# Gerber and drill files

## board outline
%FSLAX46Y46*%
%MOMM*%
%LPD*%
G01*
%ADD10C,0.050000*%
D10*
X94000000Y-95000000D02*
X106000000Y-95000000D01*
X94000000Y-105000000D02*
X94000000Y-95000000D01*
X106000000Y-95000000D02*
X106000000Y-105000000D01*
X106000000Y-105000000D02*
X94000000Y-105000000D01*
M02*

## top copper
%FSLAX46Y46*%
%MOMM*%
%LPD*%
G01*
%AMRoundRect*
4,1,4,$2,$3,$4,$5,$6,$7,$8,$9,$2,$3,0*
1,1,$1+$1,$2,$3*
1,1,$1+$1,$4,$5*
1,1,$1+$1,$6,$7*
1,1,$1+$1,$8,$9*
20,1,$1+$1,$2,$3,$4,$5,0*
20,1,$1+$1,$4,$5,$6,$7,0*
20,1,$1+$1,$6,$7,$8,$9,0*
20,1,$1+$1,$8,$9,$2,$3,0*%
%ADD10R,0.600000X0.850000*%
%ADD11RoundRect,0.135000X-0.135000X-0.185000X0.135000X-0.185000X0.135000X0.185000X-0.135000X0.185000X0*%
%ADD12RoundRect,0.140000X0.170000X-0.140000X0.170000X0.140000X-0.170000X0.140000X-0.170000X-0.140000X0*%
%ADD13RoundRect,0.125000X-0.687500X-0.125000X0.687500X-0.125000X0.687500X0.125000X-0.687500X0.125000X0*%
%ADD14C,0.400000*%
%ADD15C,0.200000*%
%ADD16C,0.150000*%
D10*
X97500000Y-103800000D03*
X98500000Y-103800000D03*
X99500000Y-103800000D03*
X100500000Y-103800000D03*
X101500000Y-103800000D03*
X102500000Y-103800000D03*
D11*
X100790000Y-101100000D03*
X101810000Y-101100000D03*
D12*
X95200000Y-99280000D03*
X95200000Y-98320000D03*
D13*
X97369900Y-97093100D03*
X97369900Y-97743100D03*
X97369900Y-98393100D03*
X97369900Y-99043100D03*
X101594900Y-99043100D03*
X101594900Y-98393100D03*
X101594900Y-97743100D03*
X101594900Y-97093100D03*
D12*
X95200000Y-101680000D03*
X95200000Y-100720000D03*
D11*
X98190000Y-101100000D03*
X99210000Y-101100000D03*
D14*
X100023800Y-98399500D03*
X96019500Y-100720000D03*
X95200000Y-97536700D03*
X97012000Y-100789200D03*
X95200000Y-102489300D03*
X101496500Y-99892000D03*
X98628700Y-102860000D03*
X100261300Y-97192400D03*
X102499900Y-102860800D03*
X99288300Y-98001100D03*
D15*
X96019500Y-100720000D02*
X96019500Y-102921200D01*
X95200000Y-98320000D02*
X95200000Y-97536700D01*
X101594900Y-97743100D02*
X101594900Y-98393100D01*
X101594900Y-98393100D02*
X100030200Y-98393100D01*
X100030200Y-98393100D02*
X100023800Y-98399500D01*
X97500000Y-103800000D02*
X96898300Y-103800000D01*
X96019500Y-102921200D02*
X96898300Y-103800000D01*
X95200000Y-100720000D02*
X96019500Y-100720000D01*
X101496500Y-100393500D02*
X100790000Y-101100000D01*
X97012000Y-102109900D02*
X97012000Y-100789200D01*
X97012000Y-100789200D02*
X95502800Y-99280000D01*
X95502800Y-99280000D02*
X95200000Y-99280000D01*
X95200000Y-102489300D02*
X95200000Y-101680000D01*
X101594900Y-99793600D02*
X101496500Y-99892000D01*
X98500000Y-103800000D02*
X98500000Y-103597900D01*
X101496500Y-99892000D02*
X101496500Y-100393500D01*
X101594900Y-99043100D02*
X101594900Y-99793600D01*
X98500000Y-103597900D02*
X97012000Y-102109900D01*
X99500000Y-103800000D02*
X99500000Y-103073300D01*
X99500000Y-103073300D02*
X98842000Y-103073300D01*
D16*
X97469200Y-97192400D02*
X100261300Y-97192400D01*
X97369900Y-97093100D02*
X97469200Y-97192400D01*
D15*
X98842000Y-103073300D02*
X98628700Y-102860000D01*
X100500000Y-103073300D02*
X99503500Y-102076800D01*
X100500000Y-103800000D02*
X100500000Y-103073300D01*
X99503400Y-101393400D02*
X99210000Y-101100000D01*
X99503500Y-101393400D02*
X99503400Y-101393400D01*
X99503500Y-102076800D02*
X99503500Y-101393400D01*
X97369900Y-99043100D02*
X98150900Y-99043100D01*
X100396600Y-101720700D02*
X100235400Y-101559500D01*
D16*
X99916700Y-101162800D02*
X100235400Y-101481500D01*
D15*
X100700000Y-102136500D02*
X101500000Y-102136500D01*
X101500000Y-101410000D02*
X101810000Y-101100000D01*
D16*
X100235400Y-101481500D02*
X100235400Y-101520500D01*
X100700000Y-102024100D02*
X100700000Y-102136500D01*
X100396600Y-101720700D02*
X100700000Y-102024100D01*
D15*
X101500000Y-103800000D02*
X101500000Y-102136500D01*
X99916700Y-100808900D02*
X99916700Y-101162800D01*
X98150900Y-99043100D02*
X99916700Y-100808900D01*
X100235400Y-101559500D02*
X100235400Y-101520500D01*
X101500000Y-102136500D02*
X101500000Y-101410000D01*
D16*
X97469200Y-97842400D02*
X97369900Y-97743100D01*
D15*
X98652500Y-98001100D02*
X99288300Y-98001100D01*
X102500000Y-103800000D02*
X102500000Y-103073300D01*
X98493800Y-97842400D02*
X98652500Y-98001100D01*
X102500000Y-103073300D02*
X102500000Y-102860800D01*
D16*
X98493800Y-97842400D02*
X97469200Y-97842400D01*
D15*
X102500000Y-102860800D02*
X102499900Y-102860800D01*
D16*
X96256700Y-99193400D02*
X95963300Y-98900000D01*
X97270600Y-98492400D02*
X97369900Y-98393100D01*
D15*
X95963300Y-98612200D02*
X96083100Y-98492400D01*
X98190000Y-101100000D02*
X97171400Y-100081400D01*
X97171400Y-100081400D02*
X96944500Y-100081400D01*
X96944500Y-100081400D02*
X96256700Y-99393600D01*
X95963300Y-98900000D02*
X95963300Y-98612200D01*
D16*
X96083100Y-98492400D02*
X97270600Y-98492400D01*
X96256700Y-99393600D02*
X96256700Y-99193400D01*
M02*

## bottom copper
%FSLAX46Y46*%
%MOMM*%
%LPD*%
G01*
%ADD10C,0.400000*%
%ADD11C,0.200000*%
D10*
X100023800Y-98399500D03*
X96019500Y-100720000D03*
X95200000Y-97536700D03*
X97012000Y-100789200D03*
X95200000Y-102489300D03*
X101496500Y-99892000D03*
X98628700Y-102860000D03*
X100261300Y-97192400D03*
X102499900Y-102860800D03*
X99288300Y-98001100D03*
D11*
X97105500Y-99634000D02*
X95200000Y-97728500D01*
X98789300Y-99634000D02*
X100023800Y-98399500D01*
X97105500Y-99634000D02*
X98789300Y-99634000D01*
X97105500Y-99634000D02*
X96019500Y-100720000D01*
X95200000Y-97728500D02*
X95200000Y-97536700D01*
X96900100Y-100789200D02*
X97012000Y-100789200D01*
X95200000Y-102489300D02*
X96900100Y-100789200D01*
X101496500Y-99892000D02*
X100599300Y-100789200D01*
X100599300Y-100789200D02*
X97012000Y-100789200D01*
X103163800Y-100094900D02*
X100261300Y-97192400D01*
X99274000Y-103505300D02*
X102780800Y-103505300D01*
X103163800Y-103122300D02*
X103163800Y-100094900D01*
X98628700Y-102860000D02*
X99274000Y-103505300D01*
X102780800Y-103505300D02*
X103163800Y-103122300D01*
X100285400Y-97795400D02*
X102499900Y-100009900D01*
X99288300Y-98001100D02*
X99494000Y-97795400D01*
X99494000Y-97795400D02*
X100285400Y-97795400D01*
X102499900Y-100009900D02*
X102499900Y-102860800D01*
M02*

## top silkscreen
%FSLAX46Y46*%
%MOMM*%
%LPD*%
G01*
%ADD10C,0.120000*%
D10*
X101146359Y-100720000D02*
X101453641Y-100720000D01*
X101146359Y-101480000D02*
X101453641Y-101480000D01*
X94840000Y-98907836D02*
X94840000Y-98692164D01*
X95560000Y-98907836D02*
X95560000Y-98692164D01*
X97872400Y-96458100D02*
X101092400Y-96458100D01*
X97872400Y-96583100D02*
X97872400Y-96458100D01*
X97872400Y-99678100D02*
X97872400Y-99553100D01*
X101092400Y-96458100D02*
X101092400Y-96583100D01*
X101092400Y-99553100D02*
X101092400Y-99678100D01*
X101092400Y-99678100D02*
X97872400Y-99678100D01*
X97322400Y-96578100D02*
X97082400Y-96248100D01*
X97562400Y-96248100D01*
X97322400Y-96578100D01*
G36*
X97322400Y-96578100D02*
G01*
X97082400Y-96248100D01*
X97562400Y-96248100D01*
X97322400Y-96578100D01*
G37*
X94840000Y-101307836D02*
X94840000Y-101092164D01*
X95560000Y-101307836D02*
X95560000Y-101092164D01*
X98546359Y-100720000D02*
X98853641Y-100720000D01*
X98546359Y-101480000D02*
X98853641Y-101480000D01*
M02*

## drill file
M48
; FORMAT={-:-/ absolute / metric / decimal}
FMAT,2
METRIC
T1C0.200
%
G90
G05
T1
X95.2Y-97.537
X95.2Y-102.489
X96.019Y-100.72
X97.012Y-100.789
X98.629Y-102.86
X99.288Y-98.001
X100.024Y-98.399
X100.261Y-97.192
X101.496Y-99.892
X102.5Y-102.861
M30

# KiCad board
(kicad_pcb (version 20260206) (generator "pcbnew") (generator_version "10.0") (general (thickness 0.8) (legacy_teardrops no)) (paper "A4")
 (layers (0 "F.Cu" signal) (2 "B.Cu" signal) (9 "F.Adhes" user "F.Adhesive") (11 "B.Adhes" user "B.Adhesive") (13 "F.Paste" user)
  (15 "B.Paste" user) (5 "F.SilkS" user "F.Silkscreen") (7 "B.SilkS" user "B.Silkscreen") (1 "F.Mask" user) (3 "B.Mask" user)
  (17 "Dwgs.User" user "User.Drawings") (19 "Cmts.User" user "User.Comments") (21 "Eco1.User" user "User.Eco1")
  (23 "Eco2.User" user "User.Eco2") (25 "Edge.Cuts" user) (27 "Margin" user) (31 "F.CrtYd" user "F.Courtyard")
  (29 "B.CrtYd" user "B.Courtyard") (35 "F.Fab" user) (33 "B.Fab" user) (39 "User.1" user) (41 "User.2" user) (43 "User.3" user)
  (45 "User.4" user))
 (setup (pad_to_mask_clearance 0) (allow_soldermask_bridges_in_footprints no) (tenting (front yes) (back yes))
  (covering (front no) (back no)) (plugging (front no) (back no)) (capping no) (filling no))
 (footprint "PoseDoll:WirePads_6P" (layer "F.Cu") (at 100 103.8)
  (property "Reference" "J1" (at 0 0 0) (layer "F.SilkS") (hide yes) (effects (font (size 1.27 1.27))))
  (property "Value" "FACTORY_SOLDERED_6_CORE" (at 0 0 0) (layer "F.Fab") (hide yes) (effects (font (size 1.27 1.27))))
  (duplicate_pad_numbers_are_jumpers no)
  (pad "1" smd rect (at -2.5 0) (size 0.6 0.85) (layers "F.Cu" "F.Mask") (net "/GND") (thermal_bridge_angle 45))
  (pad "2" smd rect (at -1.5 0) (size 0.6 0.85) (layers "F.Cu" "F.Mask") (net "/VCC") (thermal_bridge_angle 45))
  (pad "3" smd rect (at -0.5 0) (size 0.6 0.85) (layers "F.Cu" "F.Mask") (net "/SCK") (thermal_bridge_angle 45))
  (pad "4" smd rect (at 0.5 0) (size 0.6 0.85) (layers "F.Cu" "F.Mask") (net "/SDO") (thermal_bridge_angle 45))
  (pad "5" smd rect (at 1.5 0) (size 0.6 0.85) (layers "F.Cu" "F.Mask") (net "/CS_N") (thermal_bridge_angle 45))
  (pad "6" smd rect (at 2.5 0) (size 0.6 0.85) (layers "F.Cu" "F.Mask") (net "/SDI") (thermal_bridge_angle 45)))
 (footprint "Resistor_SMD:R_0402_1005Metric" (layer "F.Cu") (at 101.3 101.1)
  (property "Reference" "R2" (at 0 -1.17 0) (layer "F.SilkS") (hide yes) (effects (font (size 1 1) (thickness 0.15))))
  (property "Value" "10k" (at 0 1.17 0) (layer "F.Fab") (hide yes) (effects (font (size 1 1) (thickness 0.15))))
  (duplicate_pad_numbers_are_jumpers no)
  (fp_line (start -0.153641 -0.38) (end 0.153641 -0.38) (stroke (width 0.12) (type solid)) (layer "F.SilkS"))
  (fp_line (start -0.153641 0.38) (end 0.153641 0.38) (stroke (width 0.12) (type solid)) (layer "F.SilkS"))
  (pad "1" smd roundrect (at -0.51 0) (size 0.54 0.64) (layers "F.Cu" "F.Mask" "F.Paste") (roundrect_rratio 0.25) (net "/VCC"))
  (pad "2" smd roundrect (at 0.51 0) (size 0.54 0.64) (layers "F.Cu" "F.Mask" "F.Paste") (roundrect_rratio 0.25) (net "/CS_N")))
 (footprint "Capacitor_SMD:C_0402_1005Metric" (layer "F.Cu") (at 95.2 98.8 90)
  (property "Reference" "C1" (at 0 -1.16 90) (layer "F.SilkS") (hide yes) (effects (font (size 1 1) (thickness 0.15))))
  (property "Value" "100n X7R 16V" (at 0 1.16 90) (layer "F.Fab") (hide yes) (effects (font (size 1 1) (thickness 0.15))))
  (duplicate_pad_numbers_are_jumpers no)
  (fp_line (start -0.107836 -0.36) (end 0.107836 -0.36) (stroke (width 0.12) (type solid)) (layer "F.SilkS"))
  (fp_line (start -0.107836 0.36) (end 0.107836 0.36) (stroke (width 0.12) (type solid)) (layer "F.SilkS"))
  (pad "1" smd roundrect (at -0.48 0 90) (size 0.56 0.62) (layers "F.Cu" "F.Mask" "F.Paste") (roundrect_rratio 0.25) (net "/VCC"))
  (pad "2" smd roundrect (at 0.48 0 90) (size 0.56 0.62) (layers "F.Cu" "F.Mask" "F.Paste") (roundrect_rratio 0.25) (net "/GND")))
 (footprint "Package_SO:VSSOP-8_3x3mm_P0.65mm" (layer "F.Cu") (at 99.4824 98.0681)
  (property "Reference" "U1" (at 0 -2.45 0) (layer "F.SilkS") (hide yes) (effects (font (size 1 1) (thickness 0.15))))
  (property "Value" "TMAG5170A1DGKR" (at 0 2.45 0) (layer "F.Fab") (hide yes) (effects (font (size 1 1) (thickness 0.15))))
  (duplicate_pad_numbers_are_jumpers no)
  (fp_line (start -1.61 -1.61) (end 1.61 -1.61) (stroke (width 0.12) (type solid)) (layer "F.SilkS"))
  (fp_line (start -1.61 -1.485) (end -1.61 -1.61) (stroke (width 0.12) (type solid)) (layer "F.SilkS"))
  (fp_line (start -1.61 1.61) (end -1.61 1.485) (stroke (width 0.12) (type solid)) (layer "F.SilkS"))
  (fp_line (start 1.61 -1.61) (end 1.61 -1.485) (stroke (width 0.12) (type solid)) (layer "F.SilkS"))
  (fp_line (start 1.61 1.485) (end 1.61 1.61) (stroke (width 0.12) (type solid)) (layer "F.SilkS"))
  (fp_line (start 1.61 1.61) (end -1.61 1.61) (stroke (width 0.12) (type solid)) (layer "F.SilkS"))
  (fp_poly (pts (xy -2.16 -1.49) (xy -2.4 -1.82) (xy -1.92 -1.82)) (stroke (width 0.12) (type solid)) (fill yes) (layer "F.SilkS"))
  (pad "1" smd roundrect (at -2.1125 -0.975) (size 1.625 0.5) (layers "F.Cu" "F.Mask" "F.Paste") (roundrect_rratio 0.25) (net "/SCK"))
  (pad "2" smd roundrect (at -2.1125 -0.325) (size 1.625 0.5) (layers "F.Cu" "F.Mask" "F.Paste") (roundrect_rratio 0.25) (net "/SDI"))
  (pad "3" smd roundrect (at -2.1125 0.325) (size 1.625 0.5) (layers "F.Cu" "F.Mask" "F.Paste") (roundrect_rratio 0.25) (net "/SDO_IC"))
  (pad "4" smd roundrect (at -2.1125 0.975) (size 1.625 0.5) (layers "F.Cu" "F.Mask" "F.Paste") (roundrect_rratio 0.25) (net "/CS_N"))
  (pad "5" smd roundrect (at 2.1125 0.975) (size 1.625 0.5) (layers "F.Cu" "F.Mask" "F.Paste") (roundrect_rratio 0.25) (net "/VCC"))
  (pad "6" smd roundrect (at 2.1125 0.325) (size 1.625 0.5) (layers "F.Cu" "F.Mask" "F.Paste") (roundrect_rratio 0.25) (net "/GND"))
  (pad "7" smd roundrect (at 2.1125 -0.325) (size 1.625 0.5) (layers "F.Cu" "F.Mask" "F.Paste") (roundrect_rratio 0.25) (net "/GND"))
  (pad "8" smd roundrect (at 2.1125 -0.975) (size 1.625 0.5) (layers "F.Cu" "F.Mask" "F.Paste") (roundrect_rratio 0.25)
   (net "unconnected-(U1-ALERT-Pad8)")))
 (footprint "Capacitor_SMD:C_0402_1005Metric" (layer "F.Cu") (at 95.2 101.2 90)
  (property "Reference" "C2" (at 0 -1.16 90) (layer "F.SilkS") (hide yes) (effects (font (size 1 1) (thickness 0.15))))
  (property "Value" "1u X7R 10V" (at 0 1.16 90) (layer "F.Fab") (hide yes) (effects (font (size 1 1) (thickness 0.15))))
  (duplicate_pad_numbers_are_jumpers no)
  (fp_line (start -0.107836 -0.36) (end 0.107836 -0.36) (stroke (width 0.12) (type solid)) (layer "F.SilkS"))
  (fp_line (start -0.107836 0.36) (end 0.107836 0.36) (stroke (width 0.12) (type solid)) (layer "F.SilkS"))
  (pad "1" smd roundrect (at -0.48 0 90) (size 0.56 0.62) (layers "F.Cu" "F.Mask" "F.Paste") (roundrect_rratio 0.25) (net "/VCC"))
  (pad "2" smd roundrect (at 0.48 0 90) (size 0.56 0.62) (layers "F.Cu" "F.Mask" "F.Paste") (roundrect_rratio 0.25) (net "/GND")))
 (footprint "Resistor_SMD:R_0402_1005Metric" (layer "F.Cu") (at 98.7 101.1)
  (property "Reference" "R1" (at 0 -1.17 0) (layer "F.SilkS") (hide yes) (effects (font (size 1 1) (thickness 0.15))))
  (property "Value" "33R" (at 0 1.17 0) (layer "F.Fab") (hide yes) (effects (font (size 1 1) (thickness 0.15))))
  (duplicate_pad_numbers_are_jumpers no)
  (fp_line (start -0.153641 -0.38) (end 0.153641 -0.38) (stroke (width 0.12) (type solid)) (layer "F.SilkS"))
  (fp_line (start -0.153641 0.38) (end 0.153641 0.38) (stroke (width 0.12) (type solid)) (layer "F.SilkS"))
  (pad "1" smd roundrect (at -0.51 0) (size 0.54 0.64) (layers "F.Cu" "F.Mask" "F.Paste") (roundrect_rratio 0.25) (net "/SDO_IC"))
  (pad "2" smd roundrect (at 0.51 0) (size 0.54 0.64) (layers "F.Cu" "F.Mask" "F.Paste") (roundrect_rratio 0.25) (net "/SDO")))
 (gr_line (start 94 95) (end 106 95) (stroke (width 0.05) (type default)) (layer "Edge.Cuts"))
 (gr_line (start 94 105) (end 94 95) (stroke (width 0.05) (type default)) (layer "Edge.Cuts"))
 (gr_line (start 106 95) (end 106 105) (stroke (width 0.05) (type default)) (layer "Edge.Cuts"))
 (gr_line (start 106 105) (end 94 105) (stroke (width 0.05) (type default)) (layer "Edge.Cuts"))
 (segment (start 96.0195 100.72) (end 96.0195 102.9212) (width 0.2) (layer "F.Cu") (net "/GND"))
 (segment (start 95.2 98.32) (end 95.2 97.5367) (width 0.2) (layer "F.Cu") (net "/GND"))
 (segment (start 101.5949 97.7431) (end 101.5949 98.3931) (width 0.2) (layer "F.Cu") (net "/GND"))
 (segment (start 101.5949 98.3931) (end 100.0302 98.3931) (width 0.2) (layer "F.Cu") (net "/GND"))
 (segment (start 100.0302 98.3931) (end 100.0238 98.3995) (width 0.2) (layer "F.Cu") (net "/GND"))
 (segment (start 97.5 103.8) (end 96.8983 103.8) (width 0.2) (layer "F.Cu") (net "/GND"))
 (segment (start 96.0195 102.9212) (end 96.8983 103.8) (width 0.2) (layer "F.Cu") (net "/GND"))
 (segment (start 95.2 100.72) (end 96.0195 100.72) (width 0.2) (layer "F.Cu") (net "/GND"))
 (via (at 100.0238 98.3995) (size 0.4) (drill 0.2) (layers "F.Cu" "B.Cu") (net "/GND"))
 (via (at 96.0195 100.72) (size 0.4) (drill 0.2) (layers "F.Cu" "B.Cu") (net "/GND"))
 (via (at 95.2 97.5367) (size 0.4) (drill 0.2) (layers "F.Cu" "B.Cu") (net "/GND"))
 (segment (start 97.1055 99.634) (end 95.2 97.7285) (width 0.2) (layer "B.Cu") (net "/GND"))
 (segment (start 98.7893 99.634) (end 100.0238 98.3995) (width 0.2) (layer "B.Cu") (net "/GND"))
 (segment (start 97.1055 99.634) (end 98.7893 99.634) (width 0.2) (layer "B.Cu") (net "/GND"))
 (segment (start 97.1055 99.634) (end 96.0195 100.72) (width 0.2) (layer "B.Cu") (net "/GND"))
 (segment (start 95.2 97.7285) (end 95.2 97.5367) (width 0.2) (layer "B.Cu") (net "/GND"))
 (segment (start 101.4965 100.3935) (end 100.79 101.1) (width 0.2) (layer "F.Cu") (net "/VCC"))
 (segment (start 97.012 102.1099) (end 97.012 100.7892) (width 0.2) (layer "F.Cu") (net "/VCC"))
 (segment (start 97.012 100.7892) (end 95.5028 99.28) (width 0.2) (layer "F.Cu") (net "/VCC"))
 (segment (start 95.5028 99.28) (end 95.2 99.28) (width 0.2) (layer "F.Cu") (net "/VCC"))
 (segment (start 95.2 102.4893) (end 95.2 101.68) (width 0.2) (layer "F.Cu") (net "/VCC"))
 (segment (start 101.5949 99.7936) (end 101.4965 99.892) (width 0.2) (layer "F.Cu") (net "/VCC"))
 (segment (start 98.5 103.8) (end 98.5 103.5979) (width 0.2) (layer "F.Cu") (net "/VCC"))
 (segment (start 101.4965 99.892) (end 101.4965 100.3935) (width 0.2) (layer "F.Cu") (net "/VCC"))
 (segment (start 101.5949 99.0431) (end 101.5949 99.7936) (width 0.2) (layer "F.Cu") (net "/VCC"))
 (segment (start 98.5 103.5979) (end 97.012 102.1099) (width 0.2) (layer "F.Cu") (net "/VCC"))
 (via (at 97.012 100.7892) (size 0.4) (drill 0.2) (layers "F.Cu" "B.Cu") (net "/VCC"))
 (via (at 95.2 102.4893) (size 0.4) (drill 0.2) (layers "F.Cu" "B.Cu") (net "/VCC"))
 (via (at 101.4965 99.892) (size 0.4) (drill 0.2) (layers "F.Cu" "B.Cu") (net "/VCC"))
 (segment (start 96.9001 100.7892) (end 97.012 100.7892) (width 0.2) (layer "B.Cu") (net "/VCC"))
 (segment (start 95.2 102.4893) (end 96.9001 100.7892) (width 0.2) (layer "B.Cu") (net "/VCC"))
 (segment (start 101.4965 99.892) (end 100.5993 100.7892) (width 0.2) (layer "B.Cu") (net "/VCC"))
 (segment (start 100.5993 100.7892) (end 97.012 100.7892) (width 0.2) (layer "B.Cu") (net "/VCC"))
 (segment (start 99.5 103.8) (end 99.5 103.0733) (width 0.2) (layer "F.Cu") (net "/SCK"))
 (segment (start 99.5 103.0733) (end 98.842 103.0733) (width 0.2) (layer "F.Cu") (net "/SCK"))
 (segment (start 97.4692 97.1924) (end 100.2613 97.1924) (width 0.15) (layer "F.Cu") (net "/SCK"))
 (segment (start 97.3699 97.0931) (end 97.4692 97.1924) (width 0.15) (layer "F.Cu") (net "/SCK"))
 (segment (start 98.842 103.0733) (end 98.6287 102.86) (width 0.2) (layer "F.Cu") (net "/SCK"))
 (via (at 98.6287 102.86) (size 0.4) (drill 0.2) (layers "F.Cu" "B.Cu") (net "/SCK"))
 (via (at 100.2613 97.1924) (size 0.4) (drill 0.2) (layers "F.Cu" "B.Cu") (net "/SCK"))
 (segment (start 103.1638 100.0949) (end 100.2613 97.1924) (width 0.2) (layer "B.Cu") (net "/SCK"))
 (segment (start 99.274 103.5053) (end 102.7808 103.5053) (width 0.2) (layer "B.Cu") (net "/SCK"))
 (segment (start 103.1638 103.1223) (end 103.1638 100.0949) (width 0.2) (layer "B.Cu") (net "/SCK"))
 (segment (start 98.6287 102.86) (end 99.274 103.5053) (width 0.2) (layer "B.Cu") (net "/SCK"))
 (segment (start 102.7808 103.5053) (end 103.1638 103.1223) (width 0.2) (layer "B.Cu") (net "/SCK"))
 (segment (start 100.5 103.0733) (end 99.5035 102.0768) (width 0.2) (layer "F.Cu") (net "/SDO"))
 (segment (start 100.5 103.8) (end 100.5 103.0733) (width 0.2) (layer "F.Cu") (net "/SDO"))
 (segment (start 99.5034 101.3934) (end 99.21 101.1) (width 0.2) (layer "F.Cu") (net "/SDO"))
 (segment (start 99.5035 101.3934) (end 99.5034 101.3934) (width 0.2) (layer "F.Cu") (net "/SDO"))
 (segment (start 99.5035 102.0768) (end 99.5035 101.3934) (width 0.2) (layer "F.Cu") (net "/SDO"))
 (segment (start 97.3699 99.0431) (end 98.1509 99.0431) (width 0.2) (layer "F.Cu") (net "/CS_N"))
 (segment (start 100.3966 101.7207) (end 100.2354 101.5595) (width 0.2) (layer "F.Cu") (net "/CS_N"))
 (segment (start 99.9167 101.1628) (end 100.2354 101.4815) (width 0.15) (layer "F.Cu") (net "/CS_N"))
 (segment (start 100.7 102.1365) (end 101.5 102.1365) (width 0.2) (layer "F.Cu") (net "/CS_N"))
 (segment (start 101.5 101.41) (end 101.81 101.1) (width 0.2) (layer "F.Cu") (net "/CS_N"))
 (segment (start 100.2354 101.4815) (end 100.2354 101.5205) (width 0.15) (layer "F.Cu") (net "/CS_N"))
 (segment (start 100.7 102.0241) (end 100.7 102.1365) (width 0.15) (layer "F.Cu") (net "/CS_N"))
 (segment (start 100.3966 101.7207) (end 100.7 102.0241) (width 0.15) (layer "F.Cu") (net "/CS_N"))
 (segment (start 101.5 103.8) (end 101.5 102.1365) (width 0.2) (layer "F.Cu") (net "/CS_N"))
 (segment (start 99.9167 100.8089) (end 99.9167 101.1628) (width 0.2) (layer "F.Cu") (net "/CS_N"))
 (segment (start 98.1509 99.0431) (end 99.9167 100.8089) (width 0.2) (layer "F.Cu") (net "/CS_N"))
 (segment (start 100.2354 101.5595) (end 100.2354 101.5205) (width 0.2) (layer "F.Cu") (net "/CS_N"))
 (segment (start 101.5 102.1365) (end 101.5 101.41) (width 0.2) (layer "F.Cu") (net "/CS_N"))
 (segment (start 97.4692 97.8424) (end 97.3699 97.7431) (width 0.15) (layer "F.Cu") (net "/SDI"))
 (segment (start 98.6525 98.0011) (end 99.2883 98.0011) (width 0.2) (layer "F.Cu") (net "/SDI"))
 (segment (start 102.5 103.8) (end 102.5 103.0733) (width 0.2) (layer "F.Cu") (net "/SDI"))
 (segment (start 98.4938 97.8424) (end 98.6525 98.0011) (width 0.2) (layer "F.Cu") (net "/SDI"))
 (segment (start 102.5 103.0733) (end 102.5 102.8608) (width 0.2) (layer "F.Cu") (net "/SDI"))
 (segment (start 98.4938 97.8424) (end 97.4692 97.8424) (width 0.15) (layer "F.Cu") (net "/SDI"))
 (segment (start 102.5 102.8608) (end 102.4999 102.8608) (width 0.2) (layer "F.Cu") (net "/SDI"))
 (via (at 102.4999 102.8608) (size 0.4) (drill 0.2) (layers "F.Cu" "B.Cu") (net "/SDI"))
 (via (at 99.2883 98.0011) (size 0.4) (drill 0.2) (layers "F.Cu" "B.Cu") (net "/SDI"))
 (segment (start 100.2854 97.7954) (end 102.4999 100.0099) (width 0.2) (layer "B.Cu") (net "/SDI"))
 (segment (start 99.2883 98.0011) (end 99.494 97.7954) (width 0.2) (layer "B.Cu") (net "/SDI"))
 (segment (start 99.494 97.7954) (end 100.2854 97.7954) (width 0.2) (layer "B.Cu") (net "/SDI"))
 (segment (start 102.4999 100.0099) (end 102.4999 102.8608) (width 0.2) (layer "B.Cu") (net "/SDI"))
 (segment (start 96.2567 99.1934) (end 95.9633 98.9) (width 0.15) (layer "F.Cu") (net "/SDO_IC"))
 (segment (start 97.2706 98.4924) (end 97.3699 98.3931) (width 0.15) (layer "F.Cu") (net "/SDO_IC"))
 (segment (start 95.9633 98.6122) (end 96.0831 98.4924) (width 0.2) (layer "F.Cu") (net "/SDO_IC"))
 (segment (start 98.19 101.1) (end 97.1714 100.0814) (width 0.2) (layer "F.Cu") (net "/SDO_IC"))
 (segment (start 97.1714 100.0814) (end 96.9445 100.0814) (width 0.2) (layer "F.Cu") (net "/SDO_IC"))
 (segment (start 96.9445 100.0814) (end 96.2567 99.3936) (width 0.2) (layer "F.Cu") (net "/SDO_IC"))
 (segment (start 95.9633 98.9) (end 95.9633 98.6122) (width 0.2) (layer "F.Cu") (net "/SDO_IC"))
 (segment (start 96.0831 98.4924) (end 97.2706 98.4924) (width 0.15) (layer "F.Cu") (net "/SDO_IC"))
 (segment (start 96.2567 99.3936) (end 96.2567 99.1934) (width 0.15) (layer "F.Cu") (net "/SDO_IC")))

